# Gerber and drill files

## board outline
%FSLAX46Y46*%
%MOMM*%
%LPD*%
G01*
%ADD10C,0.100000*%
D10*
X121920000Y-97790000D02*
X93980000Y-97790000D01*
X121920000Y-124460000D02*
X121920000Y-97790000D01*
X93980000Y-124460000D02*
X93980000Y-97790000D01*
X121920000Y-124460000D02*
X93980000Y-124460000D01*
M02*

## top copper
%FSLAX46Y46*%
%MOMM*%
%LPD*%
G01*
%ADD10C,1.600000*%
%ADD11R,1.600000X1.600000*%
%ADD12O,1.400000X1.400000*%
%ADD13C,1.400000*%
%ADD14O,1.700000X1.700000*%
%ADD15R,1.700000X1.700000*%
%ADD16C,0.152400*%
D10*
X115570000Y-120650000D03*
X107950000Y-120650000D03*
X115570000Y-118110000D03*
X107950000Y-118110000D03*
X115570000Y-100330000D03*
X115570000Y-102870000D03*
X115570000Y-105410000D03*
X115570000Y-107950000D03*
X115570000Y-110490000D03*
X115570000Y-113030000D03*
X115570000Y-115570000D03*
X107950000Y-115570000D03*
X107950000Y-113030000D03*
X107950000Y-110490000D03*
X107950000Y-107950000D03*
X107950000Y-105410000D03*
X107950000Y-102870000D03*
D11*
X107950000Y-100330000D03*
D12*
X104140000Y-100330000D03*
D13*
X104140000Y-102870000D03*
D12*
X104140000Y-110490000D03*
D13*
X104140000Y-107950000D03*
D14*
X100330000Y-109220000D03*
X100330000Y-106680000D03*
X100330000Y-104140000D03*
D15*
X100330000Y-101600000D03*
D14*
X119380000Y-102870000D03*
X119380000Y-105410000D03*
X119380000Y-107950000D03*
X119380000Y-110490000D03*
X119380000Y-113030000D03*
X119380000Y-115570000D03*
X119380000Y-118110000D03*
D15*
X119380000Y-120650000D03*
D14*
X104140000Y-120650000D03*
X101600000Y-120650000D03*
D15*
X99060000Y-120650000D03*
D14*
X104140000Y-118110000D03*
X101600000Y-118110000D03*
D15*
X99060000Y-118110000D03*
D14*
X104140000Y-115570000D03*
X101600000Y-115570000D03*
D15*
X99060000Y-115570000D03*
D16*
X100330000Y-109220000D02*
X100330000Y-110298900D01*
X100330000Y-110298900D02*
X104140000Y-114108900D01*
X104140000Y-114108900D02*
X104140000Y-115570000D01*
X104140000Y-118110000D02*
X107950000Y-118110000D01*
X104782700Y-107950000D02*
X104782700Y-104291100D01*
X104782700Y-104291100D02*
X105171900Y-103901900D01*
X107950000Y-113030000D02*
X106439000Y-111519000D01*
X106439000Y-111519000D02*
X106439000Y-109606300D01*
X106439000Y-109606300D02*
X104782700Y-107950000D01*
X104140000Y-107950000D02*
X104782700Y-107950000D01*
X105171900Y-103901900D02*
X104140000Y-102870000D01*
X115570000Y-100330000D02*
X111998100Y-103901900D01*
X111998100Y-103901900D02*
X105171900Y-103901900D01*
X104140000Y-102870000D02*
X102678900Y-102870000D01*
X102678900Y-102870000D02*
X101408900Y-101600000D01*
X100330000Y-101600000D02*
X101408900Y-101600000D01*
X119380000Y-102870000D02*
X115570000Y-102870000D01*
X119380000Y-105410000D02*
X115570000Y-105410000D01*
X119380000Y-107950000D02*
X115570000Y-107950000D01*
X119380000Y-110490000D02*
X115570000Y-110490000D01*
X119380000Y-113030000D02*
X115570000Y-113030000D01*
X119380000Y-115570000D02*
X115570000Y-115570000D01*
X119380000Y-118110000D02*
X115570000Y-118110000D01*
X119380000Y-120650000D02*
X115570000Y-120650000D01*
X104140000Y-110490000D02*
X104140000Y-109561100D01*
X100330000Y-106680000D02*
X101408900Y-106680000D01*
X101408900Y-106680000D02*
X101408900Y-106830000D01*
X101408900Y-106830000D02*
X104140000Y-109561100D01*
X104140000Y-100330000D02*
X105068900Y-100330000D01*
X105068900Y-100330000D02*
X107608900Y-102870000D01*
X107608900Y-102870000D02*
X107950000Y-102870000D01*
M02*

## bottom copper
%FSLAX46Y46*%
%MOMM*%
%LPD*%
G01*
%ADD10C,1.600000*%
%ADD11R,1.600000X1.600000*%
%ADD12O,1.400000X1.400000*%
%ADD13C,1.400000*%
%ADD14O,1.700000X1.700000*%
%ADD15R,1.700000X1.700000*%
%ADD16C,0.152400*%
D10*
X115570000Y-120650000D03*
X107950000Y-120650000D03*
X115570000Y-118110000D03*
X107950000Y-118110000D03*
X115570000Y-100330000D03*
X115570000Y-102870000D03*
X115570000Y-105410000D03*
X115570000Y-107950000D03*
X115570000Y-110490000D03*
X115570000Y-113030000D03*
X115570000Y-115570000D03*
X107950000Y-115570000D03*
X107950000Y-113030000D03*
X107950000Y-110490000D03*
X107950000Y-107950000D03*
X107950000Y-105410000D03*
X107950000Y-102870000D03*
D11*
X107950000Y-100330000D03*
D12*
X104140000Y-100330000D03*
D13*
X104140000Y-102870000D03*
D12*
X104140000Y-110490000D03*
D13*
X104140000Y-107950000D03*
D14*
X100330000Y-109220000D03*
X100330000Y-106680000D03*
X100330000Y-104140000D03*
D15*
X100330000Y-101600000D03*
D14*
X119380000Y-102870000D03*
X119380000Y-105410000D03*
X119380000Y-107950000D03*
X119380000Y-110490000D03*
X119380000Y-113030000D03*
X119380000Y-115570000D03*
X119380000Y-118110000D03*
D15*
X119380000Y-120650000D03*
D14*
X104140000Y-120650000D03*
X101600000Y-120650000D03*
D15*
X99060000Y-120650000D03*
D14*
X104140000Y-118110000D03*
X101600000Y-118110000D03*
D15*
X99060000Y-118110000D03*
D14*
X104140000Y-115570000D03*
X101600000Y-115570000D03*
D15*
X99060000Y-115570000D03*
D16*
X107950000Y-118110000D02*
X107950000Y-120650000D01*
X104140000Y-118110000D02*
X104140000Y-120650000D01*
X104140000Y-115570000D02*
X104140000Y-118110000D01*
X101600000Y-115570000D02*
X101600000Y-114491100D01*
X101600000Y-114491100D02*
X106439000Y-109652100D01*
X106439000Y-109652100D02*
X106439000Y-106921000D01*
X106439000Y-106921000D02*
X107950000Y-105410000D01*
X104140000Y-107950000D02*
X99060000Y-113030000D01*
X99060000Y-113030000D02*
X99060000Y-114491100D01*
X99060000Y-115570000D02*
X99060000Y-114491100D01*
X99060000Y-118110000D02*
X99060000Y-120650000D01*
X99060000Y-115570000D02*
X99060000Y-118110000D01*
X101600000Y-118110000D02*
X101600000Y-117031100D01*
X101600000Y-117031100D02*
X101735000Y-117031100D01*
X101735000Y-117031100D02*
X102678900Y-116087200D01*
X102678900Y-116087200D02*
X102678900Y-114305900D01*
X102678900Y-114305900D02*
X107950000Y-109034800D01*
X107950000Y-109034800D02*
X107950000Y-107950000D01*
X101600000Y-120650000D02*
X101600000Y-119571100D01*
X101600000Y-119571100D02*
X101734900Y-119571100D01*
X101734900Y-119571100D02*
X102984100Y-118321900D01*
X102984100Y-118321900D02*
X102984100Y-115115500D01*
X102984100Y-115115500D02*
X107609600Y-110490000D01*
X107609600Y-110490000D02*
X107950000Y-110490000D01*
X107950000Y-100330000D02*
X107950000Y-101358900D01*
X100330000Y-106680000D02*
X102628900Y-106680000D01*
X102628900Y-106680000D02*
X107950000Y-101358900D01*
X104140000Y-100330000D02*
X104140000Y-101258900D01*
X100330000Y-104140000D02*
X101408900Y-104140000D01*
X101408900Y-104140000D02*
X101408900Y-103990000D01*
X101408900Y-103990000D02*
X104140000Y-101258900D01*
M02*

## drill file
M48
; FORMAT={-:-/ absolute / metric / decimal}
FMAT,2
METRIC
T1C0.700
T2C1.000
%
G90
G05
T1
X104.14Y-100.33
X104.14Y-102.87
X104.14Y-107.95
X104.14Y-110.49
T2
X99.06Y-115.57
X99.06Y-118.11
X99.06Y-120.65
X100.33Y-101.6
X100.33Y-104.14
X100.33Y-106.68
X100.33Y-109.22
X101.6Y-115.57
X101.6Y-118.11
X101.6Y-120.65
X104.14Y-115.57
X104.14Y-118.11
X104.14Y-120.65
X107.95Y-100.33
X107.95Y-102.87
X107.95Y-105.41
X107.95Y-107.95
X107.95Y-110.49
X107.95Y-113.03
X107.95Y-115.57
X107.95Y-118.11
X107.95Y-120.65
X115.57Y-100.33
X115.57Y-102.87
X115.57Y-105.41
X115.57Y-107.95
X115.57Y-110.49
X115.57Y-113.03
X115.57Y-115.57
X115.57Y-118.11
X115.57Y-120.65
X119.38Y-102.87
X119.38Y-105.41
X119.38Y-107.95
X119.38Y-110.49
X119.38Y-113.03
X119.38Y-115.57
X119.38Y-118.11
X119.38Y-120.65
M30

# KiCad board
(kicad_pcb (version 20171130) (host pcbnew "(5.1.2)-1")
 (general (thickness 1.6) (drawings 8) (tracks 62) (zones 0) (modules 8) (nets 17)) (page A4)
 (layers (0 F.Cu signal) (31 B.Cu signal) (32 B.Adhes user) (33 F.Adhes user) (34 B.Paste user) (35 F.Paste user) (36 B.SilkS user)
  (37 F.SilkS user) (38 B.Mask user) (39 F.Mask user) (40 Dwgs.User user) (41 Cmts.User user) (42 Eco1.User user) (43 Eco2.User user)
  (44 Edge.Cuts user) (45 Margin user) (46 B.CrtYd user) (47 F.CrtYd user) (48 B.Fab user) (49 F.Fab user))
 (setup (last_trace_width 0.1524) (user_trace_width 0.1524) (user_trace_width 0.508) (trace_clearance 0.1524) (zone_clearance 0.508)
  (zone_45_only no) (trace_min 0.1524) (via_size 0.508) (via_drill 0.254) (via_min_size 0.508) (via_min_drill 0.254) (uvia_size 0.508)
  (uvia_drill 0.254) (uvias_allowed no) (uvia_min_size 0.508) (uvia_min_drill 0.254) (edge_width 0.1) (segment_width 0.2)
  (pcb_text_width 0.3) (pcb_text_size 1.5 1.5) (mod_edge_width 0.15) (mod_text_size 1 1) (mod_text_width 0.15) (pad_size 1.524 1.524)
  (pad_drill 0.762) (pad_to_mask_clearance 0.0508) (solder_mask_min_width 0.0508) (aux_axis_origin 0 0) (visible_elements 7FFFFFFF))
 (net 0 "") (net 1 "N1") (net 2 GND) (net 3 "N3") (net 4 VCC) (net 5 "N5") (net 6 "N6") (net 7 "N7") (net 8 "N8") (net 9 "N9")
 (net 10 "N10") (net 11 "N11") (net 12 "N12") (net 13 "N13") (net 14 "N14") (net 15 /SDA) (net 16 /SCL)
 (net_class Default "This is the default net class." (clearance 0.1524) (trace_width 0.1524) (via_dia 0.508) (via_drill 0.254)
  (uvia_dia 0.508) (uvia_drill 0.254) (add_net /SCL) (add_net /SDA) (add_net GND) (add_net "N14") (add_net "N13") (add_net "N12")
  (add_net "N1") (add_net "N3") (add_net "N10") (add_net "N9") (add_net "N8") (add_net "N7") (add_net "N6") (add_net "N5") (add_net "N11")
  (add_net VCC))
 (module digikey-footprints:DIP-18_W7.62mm (layer F.Cu) (at 107.95 100.33)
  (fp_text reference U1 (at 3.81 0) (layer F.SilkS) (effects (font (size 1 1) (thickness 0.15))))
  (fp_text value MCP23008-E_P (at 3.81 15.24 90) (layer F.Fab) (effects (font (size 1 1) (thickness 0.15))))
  (pad 10 thru_hole circle (at 7.62 20.32) (size 1.6 1.6) (drill 1) (layers *.Cu *.Mask) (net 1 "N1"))
  (pad 9 thru_hole circle (at 0 20.32) (size 1.6 1.6) (drill 1) (layers *.Cu *.Mask) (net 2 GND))
  (pad 11 thru_hole circle (at 7.62 17.78) (size 1.6 1.6) (drill 1) (layers *.Cu *.Mask) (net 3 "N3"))
  (pad 8 thru_hole circle (at 0 17.78) (size 1.6 1.6) (drill 1) (layers *.Cu *.Mask) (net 2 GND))
  (pad 18 thru_hole circle (at 7.62 0) (size 1.6 1.6) (drill 1) (layers *.Cu *.Mask) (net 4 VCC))
  (pad 17 thru_hole circle (at 7.62 2.54) (size 1.6 1.6) (drill 1) (layers *.Cu *.Mask) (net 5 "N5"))
  (pad 16 thru_hole circle (at 7.62 5.08) (size 1.6 1.6) (drill 1) (layers *.Cu *.Mask) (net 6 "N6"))
  (pad 15 thru_hole circle (at 7.62 7.62) (size 1.6 1.6) (drill 1) (layers *.Cu *.Mask) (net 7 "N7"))
  (pad 14 thru_hole circle (at 7.62 10.16) (size 1.6 1.6) (drill 1) (layers *.Cu *.Mask) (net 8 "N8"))
  (pad 13 thru_hole circle (at 7.62 12.7) (size 1.6 1.6) (drill 1) (layers *.Cu *.Mask) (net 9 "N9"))
  (pad 12 thru_hole circle (at 7.62 15.24) (size 1.6 1.6) (drill 1) (layers *.Cu *.Mask) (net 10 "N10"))
  (pad 7 thru_hole circle (at 0 15.24) (size 1.6 1.6) (drill 1) (layers *.Cu *.Mask) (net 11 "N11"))
  (pad 6 thru_hole circle (at 0 12.7) (size 1.6 1.6) (drill 1) (layers *.Cu *.Mask) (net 4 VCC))
  (pad 5 thru_hole circle (at 0 10.16) (size 1.6 1.6) (drill 1) (layers *.Cu *.Mask) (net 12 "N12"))
  (pad 4 thru_hole circle (at 0 7.62) (size 1.6 1.6) (drill 1) (layers *.Cu *.Mask) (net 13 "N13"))
  (pad 3 thru_hole circle (at 0 5.08) (size 1.6 1.6) (drill 1) (layers *.Cu *.Mask) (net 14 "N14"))
  (pad 2 thru_hole circle (at 0 2.54) (size 1.6 1.6) (drill 1) (layers *.Cu *.Mask) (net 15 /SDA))
  (pad 1 thru_hole rect (at 0 0) (size 1.6 1.6) (drill 1) (layers *.Cu *.Mask) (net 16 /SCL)))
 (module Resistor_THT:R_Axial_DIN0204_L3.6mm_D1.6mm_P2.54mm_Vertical (layer F.Cu) (at 104.14 102.87 90)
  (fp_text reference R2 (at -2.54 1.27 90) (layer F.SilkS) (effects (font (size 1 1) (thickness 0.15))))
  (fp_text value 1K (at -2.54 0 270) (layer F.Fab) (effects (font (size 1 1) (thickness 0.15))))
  (pad 2 thru_hole oval (at 2.54 0 90) (size 1.4 1.4) (drill 0.7) (layers *.Cu *.Mask) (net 15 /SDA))
  (pad 1 thru_hole circle (at 0 0 90) (size 1.4 1.4) (drill 0.7) (layers *.Cu *.Mask) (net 4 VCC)))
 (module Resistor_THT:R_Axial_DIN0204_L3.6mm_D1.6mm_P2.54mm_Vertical (layer F.Cu) (at 104.14 107.95 270)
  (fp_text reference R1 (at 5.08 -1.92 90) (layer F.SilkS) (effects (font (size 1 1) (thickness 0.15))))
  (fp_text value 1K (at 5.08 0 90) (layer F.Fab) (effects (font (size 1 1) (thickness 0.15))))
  (pad 2 thru_hole oval (at 2.54 0 270) (size 1.4 1.4) (drill 0.7) (layers *.Cu *.Mask) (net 16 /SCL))
  (pad 1 thru_hole circle (at 0 0 270) (size 1.4 1.4) (drill 0.7) (layers *.Cu *.Mask) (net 4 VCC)))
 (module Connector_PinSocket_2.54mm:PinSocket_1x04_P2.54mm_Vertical (layer F.Cu) (at 100.33 101.6)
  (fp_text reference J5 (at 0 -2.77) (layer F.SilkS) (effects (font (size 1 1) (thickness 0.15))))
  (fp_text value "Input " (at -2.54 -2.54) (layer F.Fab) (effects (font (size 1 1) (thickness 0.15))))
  (pad 4 thru_hole oval (at 0 7.62) (size 1.7 1.7) (drill 1) (layers *.Cu *.Mask) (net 2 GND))
  (pad 3 thru_hole oval (at 0 5.08) (size 1.7 1.7) (drill 1) (layers *.Cu *.Mask) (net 16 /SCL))
  (pad 2 thru_hole oval (at 0 2.54) (size 1.7 1.7) (drill 1) (layers *.Cu *.Mask) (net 15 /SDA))
  (pad 1 thru_hole rect (at 0 0) (size 1.7 1.7) (drill 1) (layers *.Cu *.Mask) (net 4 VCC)))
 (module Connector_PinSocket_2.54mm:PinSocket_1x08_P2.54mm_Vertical (layer F.Cu) (at 119.38 120.65 180)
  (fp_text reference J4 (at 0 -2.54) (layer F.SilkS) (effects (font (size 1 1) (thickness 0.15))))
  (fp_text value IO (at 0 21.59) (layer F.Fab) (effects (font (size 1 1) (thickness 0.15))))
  (pad 8 thru_hole oval (at 0 17.78 180) (size 1.7 1.7) (drill 1) (layers *.Cu *.Mask) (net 5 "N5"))
  (pad 7 thru_hole oval (at 0 15.24 180) (size 1.7 1.7) (drill 1) (layers *.Cu *.Mask) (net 6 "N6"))
  (pad 6 thru_hole oval (at 0 12.7 180) (size 1.7 1.7) (drill 1) (layers *.Cu *.Mask) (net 7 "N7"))
  (pad 5 thru_hole oval (at 0 10.16 180) (size 1.7 1.7) (drill 1) (layers *.Cu *.Mask) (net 8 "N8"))
  (pad 4 thru_hole oval (at 0 7.62 180) (size 1.7 1.7) (drill 1) (layers *.Cu *.Mask) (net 9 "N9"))
  (pad 3 thru_hole oval (at 0 5.08 180) (size 1.7 1.7) (drill 1) (layers *.Cu *.Mask) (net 10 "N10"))
  (pad 2 thru_hole oval (at 0 2.54 180) (size 1.7 1.7) (drill 1) (layers *.Cu *.Mask) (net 3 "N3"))
  (pad 1 thru_hole rect (at 0 0 180) (size 1.7 1.7) (drill 1) (layers *.Cu *.Mask) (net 1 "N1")))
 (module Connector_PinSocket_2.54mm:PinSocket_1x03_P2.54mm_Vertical (layer F.Cu) (at 99.06 120.65 90)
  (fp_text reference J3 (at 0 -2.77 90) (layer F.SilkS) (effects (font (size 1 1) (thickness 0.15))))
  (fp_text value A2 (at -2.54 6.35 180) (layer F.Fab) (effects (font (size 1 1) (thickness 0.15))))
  (pad 3 thru_hole oval (at 0 5.08 90) (size 1.7 1.7) (drill 1) (layers *.Cu *.Mask) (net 2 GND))
  (pad 2 thru_hole oval (at 0 2.54 90) (size 1.7 1.7) (drill 1) (layers *.Cu *.Mask) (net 12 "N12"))
  (pad 1 thru_hole rect (at 0 0 90) (size 1.7 1.7) (drill 1) (layers *.Cu *.Mask) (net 4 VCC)))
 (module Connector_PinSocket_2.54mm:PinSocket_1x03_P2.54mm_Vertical (layer F.Cu) (at 99.06 118.11 90)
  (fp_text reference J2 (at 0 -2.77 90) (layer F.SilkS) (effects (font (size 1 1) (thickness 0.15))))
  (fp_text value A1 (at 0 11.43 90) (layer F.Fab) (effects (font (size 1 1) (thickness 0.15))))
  (pad 3 thru_hole oval (at 0 5.08 90) (size 1.7 1.7) (drill 1) (layers *.Cu *.Mask) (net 2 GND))
  (pad 2 thru_hole oval (at 0 2.54 90) (size 1.7 1.7) (drill 1) (layers *.Cu *.Mask) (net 13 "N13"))
  (pad 1 thru_hole rect (at 0 0 90) (size 1.7 1.7) (drill 1) (layers *.Cu *.Mask) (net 4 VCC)))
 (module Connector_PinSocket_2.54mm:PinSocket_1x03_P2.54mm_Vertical (layer F.Cu) (at 99.06 115.57 90)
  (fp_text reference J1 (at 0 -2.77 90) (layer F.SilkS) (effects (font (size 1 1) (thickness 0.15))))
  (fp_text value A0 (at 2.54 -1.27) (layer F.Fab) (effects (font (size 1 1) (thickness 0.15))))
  (pad 3 thru_hole oval (at 0 5.08 90) (size 1.7 1.7) (drill 1) (layers *.Cu *.Mask) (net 2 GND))
  (pad 2 thru_hole oval (at 0 2.54 90) (size 1.7 1.7) (drill 1) (layers *.Cu *.Mask) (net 14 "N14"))
  (pad 1 thru_hole rect (at 0 0 90) (size 1.7 1.7) (drill 1) (layers *.Cu *.Mask) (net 4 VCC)))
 (gr_line (start 121.92 97.79) (end 93.98 97.79) (layer Edge.Cuts) (width 0.1))
 (gr_line (start 121.92 124.46) (end 121.92 97.79) (layer Edge.Cuts) (width 0.1))
 (gr_line (start 93.98 124.46) (end 93.98 97.79) (layer Edge.Cuts) (width 0.1))
 (gr_line (start 121.92 124.46) (end 93.98 124.46) (layer Edge.Cuts) (width 0.1))
 (segment (start 107.95 118.11) (end 107.95 120.65) (width 0.1524) (layer B.Cu) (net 2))
 (segment (start 100.33 109.22) (end 100.33 110.2989) (width 0.1524) (layer F.Cu) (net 2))
 (segment (start 100.33 110.2989) (end 104.14 114.1089) (width 0.1524) (layer F.Cu) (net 2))
 (segment (start 104.14 114.1089) (end 104.14 115.57) (width 0.1524) (layer F.Cu) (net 2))
 (segment (start 104.14 118.11) (end 107.95 118.11) (width 0.1524) (layer F.Cu) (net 2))
 (segment (start 104.14 118.11) (end 104.14 120.65) (width 0.1524) (layer B.Cu) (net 2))
 (segment (start 104.14 115.57) (end 104.14 118.11) (width 0.1524) (layer B.Cu) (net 2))
 (segment (start 101.6 115.57) (end 101.6 114.4911) (width 0.1524) (layer B.Cu) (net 14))
 (segment (start 101.6 114.4911) (end 106.439 109.6521) (width 0.1524) (layer B.Cu) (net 14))
 (segment (start 106.439 109.6521) (end 106.439 106.921) (width 0.1524) (layer B.Cu) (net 14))
 (segment (start 106.439 106.921) (end 107.95 105.41) (width 0.1524) (layer B.Cu) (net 14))
 (segment (start 104.7827 107.95) (end 104.7827 104.2911) (width 0.1524) (layer F.Cu) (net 4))
 (segment (start 104.7827 104.2911) (end 105.1719 103.9019) (width 0.1524) (layer F.Cu) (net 4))
 (segment (start 107.95 113.03) (end 106.439 111.519) (width 0.1524) (layer F.Cu) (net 4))
 (segment (start 106.439 111.519) (end 106.439 109.6063) (width 0.1524) (layer F.Cu) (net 4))
 (segment (start 106.439 109.6063) (end 104.7827 107.95) (width 0.1524) (layer F.Cu) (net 4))
 (segment (start 104.14 107.95) (end 104.7827 107.95) (width 0.1524) (layer F.Cu) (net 4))
 (segment (start 105.1719 103.9019) (end 104.14 102.87) (width 0.1524) (layer F.Cu) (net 4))
 (segment (start 115.57 100.33) (end 111.9981 103.9019) (width 0.1524) (layer F.Cu) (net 4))
 (segment (start 111.9981 103.9019) (end 105.1719 103.9019) (width 0.1524) (layer F.Cu) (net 4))
 (segment (start 104.14 102.87) (end 102.6789 102.87) (width 0.1524) (layer F.Cu) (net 4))
 (segment (start 102.6789 102.87) (end 101.4089 101.6) (width 0.1524) (layer F.Cu) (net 4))
 (segment (start 100.33 101.6) (end 101.4089 101.6) (width 0.1524) (layer F.Cu) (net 4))
 (segment (start 104.14 107.95) (end 99.06 113.03) (width 0.1524) (layer B.Cu) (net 4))
 (segment (start 99.06 113.03) (end 99.06 114.4911) (width 0.1524) (layer B.Cu) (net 4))
 (segment (start 99.06 115.57) (end 99.06 114.4911) (width 0.1524) (layer B.Cu) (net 4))
 (segment (start 99.06 118.11) (end 99.06 120.65) (width 0.1524) (layer B.Cu) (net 4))
 (segment (start 99.06 115.57) (end 99.06 118.11) (width 0.1524) (layer B.Cu) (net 4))
 (segment (start 101.6 118.11) (end 101.6 117.0311) (width 0.1524) (layer B.Cu) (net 13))
 (segment (start 101.6 117.0311) (end 101.735 117.0311) (width 0.1524) (layer B.Cu) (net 13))
 (segment (start 101.735 117.0311) (end 102.6789 116.0872) (width 0.1524) (layer B.Cu) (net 13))
 (segment (start 102.6789 116.0872) (end 102.6789 114.3059) (width 0.1524) (layer B.Cu) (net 13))
 (segment (start 102.6789 114.3059) (end 107.95 109.0348) (width 0.1524) (layer B.Cu) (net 13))
 (segment (start 107.95 109.0348) (end 107.95 107.95) (width 0.1524) (layer B.Cu) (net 13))
 (segment (start 101.6 120.65) (end 101.6 119.5711) (width 0.1524) (layer B.Cu) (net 12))
 (segment (start 101.6 119.5711) (end 101.7349 119.5711) (width 0.1524) (layer B.Cu) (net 12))
 (segment (start 101.7349 119.5711) (end 102.9841 118.3219) (width 0.1524) (layer B.Cu) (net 12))
 (segment (start 102.9841 118.3219) (end 102.9841 115.1155) (width 0.1524) (layer B.Cu) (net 12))
 (segment (start 102.9841 115.1155) (end 107.6096 110.49) (width 0.1524) (layer B.Cu) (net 12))
 (segment (start 107.6096 110.49) (end 107.95 110.49) (width 0.1524) (layer B.Cu) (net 12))
 (segment (start 119.38 102.87) (end 115.57 102.87) (width 0.1524) (layer F.Cu) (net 5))
 (segment (start 119.38 105.41) (end 115.57 105.41) (width 0.1524) (layer F.Cu) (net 6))
 (segment (start 119.38 107.95) (end 115.57 107.95) (width 0.1524) (layer F.Cu) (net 7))
 (segment (start 119.38 110.49) (end 115.57 110.49) (width 0.1524) (layer F.Cu) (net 8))
 (segment (start 119.38 113.03) (end 115.57 113.03) (width 0.1524) (layer F.Cu) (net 9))
 (segment (start 119.38 115.57) (end 115.57 115.57) (width 0.1524) (layer F.Cu) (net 10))
 (segment (start 119.38 118.11) (end 115.57 118.11) (width 0.1524) (layer F.Cu) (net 3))
 (segment (start 119.38 120.65) (end 115.57 120.65) (width 0.1524) (layer F.Cu) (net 1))
 (segment (start 107.95 100.33) (end 107.95 101.3589) (width 0.1524) (layer B.Cu) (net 16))
 (segment (start 100.33 106.68) (end 102.6289 106.68) (width 0.1524) (layer B.Cu) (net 16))
 (segment (start 102.6289 106.68) (end 107.95 101.3589) (width 0.1524) (layer B.Cu) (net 16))
 (segment (start 104.14 110.49) (end 104.14 109.5611) (width 0.1524) (layer F.Cu) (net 16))
 (segment (start 100.33 106.68) (end 101.4089 106.68) (width 0.1524) (layer F.Cu) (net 16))
 (segment (start 101.4089 106.68) (end 101.4089 106.83) (width 0.1524) (layer F.Cu) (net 16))
 (segment (start 101.4089 106.83) (end 104.14 109.5611) (width 0.1524) (layer F.Cu) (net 16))
 (segment (start 104.14 100.33) (end 105.0689 100.33) (width 0.1524) (layer F.Cu) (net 15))
 (segment (start 105.0689 100.33) (end 107.6089 102.87) (width 0.1524) (layer F.Cu) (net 15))
 (segment (start 107.6089 102.87) (end 107.95 102.87) (width 0.1524) (layer F.Cu) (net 15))
 (segment (start 104.14 100.33) (end 104.14 101.2589) (width 0.1524) (layer B.Cu) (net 15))
 (segment (start 100.33 104.14) (end 101.4089 104.14) (width 0.1524) (layer B.Cu) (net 15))
 (segment (start 101.4089 104.14) (end 101.4089 103.99) (width 0.1524) (layer B.Cu) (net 15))
 (segment (start 101.4089 103.99) (end 104.14 101.2589) (width 0.1524) (layer B.Cu) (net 15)))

